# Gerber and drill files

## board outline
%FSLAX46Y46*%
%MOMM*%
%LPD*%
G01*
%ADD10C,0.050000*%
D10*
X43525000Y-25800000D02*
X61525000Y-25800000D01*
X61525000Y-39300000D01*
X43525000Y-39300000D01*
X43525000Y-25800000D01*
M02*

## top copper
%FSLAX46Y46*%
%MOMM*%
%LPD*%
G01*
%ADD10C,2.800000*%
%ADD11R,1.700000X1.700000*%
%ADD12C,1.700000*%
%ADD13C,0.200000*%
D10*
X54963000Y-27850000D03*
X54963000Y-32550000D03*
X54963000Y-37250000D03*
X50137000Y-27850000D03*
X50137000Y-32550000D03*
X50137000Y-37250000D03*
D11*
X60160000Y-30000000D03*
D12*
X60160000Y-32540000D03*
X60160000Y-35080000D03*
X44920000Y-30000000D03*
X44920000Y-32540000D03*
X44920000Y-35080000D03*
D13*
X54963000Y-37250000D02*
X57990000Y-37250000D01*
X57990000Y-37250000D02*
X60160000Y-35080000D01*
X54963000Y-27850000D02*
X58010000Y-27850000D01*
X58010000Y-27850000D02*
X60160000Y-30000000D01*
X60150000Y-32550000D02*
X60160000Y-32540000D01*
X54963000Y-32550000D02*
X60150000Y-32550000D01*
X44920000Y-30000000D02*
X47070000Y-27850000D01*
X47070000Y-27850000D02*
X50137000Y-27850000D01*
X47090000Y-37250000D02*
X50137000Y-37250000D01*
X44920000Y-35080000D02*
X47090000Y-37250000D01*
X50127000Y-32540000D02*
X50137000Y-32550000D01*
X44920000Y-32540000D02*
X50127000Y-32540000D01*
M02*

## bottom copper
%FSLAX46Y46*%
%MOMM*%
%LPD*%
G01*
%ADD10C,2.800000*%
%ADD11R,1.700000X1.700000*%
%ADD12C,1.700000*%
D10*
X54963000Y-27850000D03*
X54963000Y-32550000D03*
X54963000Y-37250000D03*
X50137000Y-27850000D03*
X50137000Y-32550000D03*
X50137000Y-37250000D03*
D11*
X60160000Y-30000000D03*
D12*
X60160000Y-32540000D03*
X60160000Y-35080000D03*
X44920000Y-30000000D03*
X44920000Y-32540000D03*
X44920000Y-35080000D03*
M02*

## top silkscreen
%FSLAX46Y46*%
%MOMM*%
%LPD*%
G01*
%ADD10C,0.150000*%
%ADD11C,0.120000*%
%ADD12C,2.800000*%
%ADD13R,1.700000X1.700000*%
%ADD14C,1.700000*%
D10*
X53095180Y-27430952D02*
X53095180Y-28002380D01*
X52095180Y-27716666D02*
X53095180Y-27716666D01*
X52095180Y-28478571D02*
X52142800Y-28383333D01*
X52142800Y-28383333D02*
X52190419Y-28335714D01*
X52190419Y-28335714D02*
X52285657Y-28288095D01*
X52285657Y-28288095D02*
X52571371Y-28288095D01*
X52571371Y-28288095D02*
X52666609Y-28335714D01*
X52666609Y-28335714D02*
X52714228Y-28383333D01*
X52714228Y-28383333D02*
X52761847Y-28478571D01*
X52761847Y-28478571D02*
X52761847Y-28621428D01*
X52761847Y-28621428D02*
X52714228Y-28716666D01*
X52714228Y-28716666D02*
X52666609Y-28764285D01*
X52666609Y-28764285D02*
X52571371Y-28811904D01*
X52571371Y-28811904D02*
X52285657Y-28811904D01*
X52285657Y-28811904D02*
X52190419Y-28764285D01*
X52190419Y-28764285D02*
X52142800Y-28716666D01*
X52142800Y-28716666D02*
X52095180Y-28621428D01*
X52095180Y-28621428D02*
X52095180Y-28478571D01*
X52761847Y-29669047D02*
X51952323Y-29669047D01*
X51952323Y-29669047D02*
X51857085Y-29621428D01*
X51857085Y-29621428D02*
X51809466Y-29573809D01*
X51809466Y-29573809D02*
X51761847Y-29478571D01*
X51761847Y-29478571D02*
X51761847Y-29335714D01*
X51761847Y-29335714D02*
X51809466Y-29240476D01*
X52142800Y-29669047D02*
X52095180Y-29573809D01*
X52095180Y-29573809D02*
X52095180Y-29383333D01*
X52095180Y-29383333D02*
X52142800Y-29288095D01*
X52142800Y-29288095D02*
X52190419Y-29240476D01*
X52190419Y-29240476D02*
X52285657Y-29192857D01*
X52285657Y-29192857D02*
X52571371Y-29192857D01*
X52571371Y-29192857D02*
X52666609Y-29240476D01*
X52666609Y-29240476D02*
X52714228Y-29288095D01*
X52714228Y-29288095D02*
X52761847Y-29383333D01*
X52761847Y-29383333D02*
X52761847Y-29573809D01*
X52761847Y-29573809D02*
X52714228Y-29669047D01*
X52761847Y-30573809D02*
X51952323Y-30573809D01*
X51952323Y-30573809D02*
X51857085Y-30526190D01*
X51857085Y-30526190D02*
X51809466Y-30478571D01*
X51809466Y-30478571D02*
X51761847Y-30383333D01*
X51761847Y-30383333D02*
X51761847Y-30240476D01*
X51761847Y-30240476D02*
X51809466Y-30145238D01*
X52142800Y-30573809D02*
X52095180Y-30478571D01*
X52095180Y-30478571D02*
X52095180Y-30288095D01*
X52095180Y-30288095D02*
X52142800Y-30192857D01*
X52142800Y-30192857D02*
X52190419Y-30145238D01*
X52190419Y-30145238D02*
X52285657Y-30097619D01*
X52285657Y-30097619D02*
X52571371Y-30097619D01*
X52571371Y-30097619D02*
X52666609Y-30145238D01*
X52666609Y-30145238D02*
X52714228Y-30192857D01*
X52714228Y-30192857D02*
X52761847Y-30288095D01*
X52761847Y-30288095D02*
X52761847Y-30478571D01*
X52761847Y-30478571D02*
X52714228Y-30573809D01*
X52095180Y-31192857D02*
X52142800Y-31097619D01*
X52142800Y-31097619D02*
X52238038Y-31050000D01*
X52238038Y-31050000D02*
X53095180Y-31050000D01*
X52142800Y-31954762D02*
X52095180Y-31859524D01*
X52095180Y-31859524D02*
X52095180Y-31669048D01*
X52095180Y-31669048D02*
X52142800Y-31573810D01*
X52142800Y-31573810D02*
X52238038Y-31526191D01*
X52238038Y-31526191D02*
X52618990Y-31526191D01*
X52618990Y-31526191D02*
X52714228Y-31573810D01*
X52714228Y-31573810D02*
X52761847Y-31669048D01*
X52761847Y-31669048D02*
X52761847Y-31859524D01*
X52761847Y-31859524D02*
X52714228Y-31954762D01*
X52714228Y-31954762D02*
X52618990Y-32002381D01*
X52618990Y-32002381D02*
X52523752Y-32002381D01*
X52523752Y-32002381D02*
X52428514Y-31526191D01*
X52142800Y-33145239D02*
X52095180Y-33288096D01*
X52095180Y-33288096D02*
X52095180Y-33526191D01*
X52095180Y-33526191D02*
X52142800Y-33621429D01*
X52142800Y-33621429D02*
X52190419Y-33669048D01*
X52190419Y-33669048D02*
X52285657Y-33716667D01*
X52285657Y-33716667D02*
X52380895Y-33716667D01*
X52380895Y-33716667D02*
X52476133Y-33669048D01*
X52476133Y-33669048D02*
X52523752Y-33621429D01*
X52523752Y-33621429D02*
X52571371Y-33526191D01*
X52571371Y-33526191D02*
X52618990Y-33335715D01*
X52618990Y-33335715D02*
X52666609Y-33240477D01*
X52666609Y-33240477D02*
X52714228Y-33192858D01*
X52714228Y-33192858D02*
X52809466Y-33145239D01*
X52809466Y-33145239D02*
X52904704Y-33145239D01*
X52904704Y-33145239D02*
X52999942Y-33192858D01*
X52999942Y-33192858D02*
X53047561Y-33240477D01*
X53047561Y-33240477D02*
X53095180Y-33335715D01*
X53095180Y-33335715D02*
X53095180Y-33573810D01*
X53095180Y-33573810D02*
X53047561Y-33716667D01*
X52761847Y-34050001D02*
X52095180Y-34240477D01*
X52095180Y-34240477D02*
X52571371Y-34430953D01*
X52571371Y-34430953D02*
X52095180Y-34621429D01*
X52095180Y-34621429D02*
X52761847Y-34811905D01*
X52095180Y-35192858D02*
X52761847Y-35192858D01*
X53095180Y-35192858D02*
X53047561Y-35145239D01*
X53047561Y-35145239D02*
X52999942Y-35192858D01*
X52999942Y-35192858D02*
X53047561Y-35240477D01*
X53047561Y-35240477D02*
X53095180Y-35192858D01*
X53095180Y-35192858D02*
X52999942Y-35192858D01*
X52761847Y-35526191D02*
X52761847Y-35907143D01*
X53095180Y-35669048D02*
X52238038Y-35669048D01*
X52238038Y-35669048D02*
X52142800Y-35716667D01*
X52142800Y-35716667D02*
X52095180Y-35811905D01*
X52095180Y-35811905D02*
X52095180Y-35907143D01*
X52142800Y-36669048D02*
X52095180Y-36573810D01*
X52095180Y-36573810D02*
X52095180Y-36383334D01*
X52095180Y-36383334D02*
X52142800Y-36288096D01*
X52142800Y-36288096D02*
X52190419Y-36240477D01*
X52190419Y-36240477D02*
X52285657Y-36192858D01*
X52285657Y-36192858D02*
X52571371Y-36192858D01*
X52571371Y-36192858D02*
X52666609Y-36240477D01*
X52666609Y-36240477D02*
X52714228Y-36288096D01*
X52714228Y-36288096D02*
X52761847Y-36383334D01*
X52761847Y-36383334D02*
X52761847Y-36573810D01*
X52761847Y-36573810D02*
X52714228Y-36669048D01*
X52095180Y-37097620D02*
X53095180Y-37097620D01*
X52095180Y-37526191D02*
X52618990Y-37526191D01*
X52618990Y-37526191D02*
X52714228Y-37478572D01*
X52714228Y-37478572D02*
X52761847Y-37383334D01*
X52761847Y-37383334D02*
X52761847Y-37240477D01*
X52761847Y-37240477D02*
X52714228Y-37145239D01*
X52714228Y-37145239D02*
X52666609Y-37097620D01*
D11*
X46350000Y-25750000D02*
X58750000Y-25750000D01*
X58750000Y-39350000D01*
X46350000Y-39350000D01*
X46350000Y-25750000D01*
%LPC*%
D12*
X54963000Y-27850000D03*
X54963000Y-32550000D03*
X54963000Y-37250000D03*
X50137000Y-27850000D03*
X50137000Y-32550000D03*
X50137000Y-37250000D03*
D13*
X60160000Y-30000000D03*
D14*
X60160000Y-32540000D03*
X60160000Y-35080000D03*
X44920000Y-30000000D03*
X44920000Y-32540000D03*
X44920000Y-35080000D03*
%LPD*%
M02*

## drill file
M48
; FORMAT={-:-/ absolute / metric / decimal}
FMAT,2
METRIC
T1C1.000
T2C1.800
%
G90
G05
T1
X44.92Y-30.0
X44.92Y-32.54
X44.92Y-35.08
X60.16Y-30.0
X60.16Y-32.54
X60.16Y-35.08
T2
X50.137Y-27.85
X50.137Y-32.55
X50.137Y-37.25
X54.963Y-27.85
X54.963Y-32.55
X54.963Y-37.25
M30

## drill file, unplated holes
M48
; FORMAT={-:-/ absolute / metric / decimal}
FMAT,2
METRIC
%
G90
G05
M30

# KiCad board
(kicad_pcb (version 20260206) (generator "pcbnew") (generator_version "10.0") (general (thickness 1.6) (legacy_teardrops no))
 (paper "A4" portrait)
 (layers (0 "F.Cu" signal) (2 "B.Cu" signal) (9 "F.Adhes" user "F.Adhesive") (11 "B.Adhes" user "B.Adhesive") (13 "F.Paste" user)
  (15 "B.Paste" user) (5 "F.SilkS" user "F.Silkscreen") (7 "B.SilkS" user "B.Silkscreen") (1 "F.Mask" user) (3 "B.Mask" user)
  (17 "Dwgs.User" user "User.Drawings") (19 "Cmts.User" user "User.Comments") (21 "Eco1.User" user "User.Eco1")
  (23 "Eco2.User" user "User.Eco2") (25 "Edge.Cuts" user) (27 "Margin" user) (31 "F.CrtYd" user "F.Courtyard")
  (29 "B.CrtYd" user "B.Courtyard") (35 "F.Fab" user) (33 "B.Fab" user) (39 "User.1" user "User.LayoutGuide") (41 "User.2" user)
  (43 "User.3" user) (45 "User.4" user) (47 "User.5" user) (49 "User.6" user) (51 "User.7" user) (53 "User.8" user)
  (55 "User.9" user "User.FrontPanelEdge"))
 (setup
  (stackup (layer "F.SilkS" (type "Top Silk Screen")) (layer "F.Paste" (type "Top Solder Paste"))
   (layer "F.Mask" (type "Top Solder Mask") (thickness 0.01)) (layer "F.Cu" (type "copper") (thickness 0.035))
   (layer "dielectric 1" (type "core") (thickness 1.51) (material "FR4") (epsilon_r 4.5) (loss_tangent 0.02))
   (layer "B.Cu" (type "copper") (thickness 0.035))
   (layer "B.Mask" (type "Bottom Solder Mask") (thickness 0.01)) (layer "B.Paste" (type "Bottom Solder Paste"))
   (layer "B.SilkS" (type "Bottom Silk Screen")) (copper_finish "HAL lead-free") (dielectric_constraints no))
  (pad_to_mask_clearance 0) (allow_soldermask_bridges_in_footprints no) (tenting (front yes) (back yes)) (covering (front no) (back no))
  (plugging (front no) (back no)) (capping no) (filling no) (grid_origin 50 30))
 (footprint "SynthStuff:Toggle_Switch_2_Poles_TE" (layer "F.Cu") (at 52.55 32.55 180)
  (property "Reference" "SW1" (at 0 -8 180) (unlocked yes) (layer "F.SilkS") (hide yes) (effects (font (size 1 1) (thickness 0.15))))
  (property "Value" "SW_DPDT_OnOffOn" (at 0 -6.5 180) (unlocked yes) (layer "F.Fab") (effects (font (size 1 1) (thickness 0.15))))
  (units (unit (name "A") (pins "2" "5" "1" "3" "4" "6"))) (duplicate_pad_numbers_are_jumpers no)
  (fp_rect (start -6.2 -6.8) (end 6.2 6.8) (stroke (width 0.12) (type default)) (fill no) (layer "F.SilkS"))
  (pad "1" thru_hole circle (at -2.413 4.7 270) (size 2.8 2.8) (drill 1.8) (layers "*.Cu" "*.Mask") (remove_unused_layers no)
   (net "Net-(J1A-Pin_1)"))
  (pad "2" thru_hole circle (at -2.413 0 270) (size 2.8 2.8) (drill 1.8) (layers "*.Cu" "*.Mask") (remove_unused_layers no)
   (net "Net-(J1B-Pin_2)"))
  (pad "3" thru_hole circle (at -2.413 -4.7 270) (size 2.8 2.8) (drill 1.8) (layers "*.Cu" "*.Mask") (remove_unused_layers no)
   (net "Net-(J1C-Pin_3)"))
  (pad "4" thru_hole circle (at 2.413 4.7 270) (size 2.8 2.8) (drill 1.8) (layers "*.Cu" "*.Mask") (remove_unused_layers no)
   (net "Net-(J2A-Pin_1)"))
  (pad "5" thru_hole circle (at 2.413 0 270) (size 2.8 2.8) (drill 1.8) (layers "*.Cu" "*.Mask") (remove_unused_layers no)
   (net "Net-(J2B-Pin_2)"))
  (pad "6" thru_hole circle (at 2.413 -4.7 270) (size 2.8 2.8) (drill 1.8) (layers "*.Cu" "*.Mask") (remove_unused_layers no)
   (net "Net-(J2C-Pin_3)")))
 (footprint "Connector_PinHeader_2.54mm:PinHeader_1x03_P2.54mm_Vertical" (layer "B.Cu") (at 60.16 30 180)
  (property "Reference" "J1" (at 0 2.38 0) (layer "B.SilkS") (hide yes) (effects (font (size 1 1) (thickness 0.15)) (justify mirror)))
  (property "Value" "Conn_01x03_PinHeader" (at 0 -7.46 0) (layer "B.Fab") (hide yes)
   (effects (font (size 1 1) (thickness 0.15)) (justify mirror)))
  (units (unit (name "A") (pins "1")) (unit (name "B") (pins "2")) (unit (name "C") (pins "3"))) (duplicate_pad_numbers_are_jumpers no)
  (pad "1" thru_hole rect (at 0 0 180) (size 1.7 1.7) (drill 1) (layers "*.Cu" "*.Mask") (remove_unused_layers no) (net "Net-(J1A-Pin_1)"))
  (pad "2" thru_hole circle (at 0 -2.54 180) (size 1.7 1.7) (drill 1) (layers "*.Cu" "*.Mask") (remove_unused_layers no)
   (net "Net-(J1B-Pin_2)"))
  (pad "3" thru_hole circle (at 0 -5.08 180) (size 1.7 1.7) (drill 1) (layers "*.Cu" "*.Mask") (remove_unused_layers no)
   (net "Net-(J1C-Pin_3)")))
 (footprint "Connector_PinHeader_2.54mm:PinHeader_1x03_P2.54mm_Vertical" (layer "B.Cu") (at 44.92 30 180)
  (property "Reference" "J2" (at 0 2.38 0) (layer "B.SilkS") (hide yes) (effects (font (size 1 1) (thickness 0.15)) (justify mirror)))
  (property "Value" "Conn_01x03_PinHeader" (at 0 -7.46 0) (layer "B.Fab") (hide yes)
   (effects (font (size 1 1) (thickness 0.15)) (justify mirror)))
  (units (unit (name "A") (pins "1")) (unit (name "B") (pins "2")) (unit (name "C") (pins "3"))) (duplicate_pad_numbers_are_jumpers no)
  (pad "1" thru_hole circle (at 0 0 180) (size 1.7 1.7) (drill 1) (layers "*.Cu" "*.Mask") (remove_unused_layers no) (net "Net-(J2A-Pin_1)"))
  (pad "2" thru_hole circle (at 0 -2.54 180) (size 1.7 1.7) (drill 1) (layers "*.Cu" "*.Mask") (remove_unused_layers no)
   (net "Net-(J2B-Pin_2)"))
  (pad "3" thru_hole circle (at 0 -5.08 180) (size 1.7 1.7) (drill 1) (layers "*.Cu" "*.Mask") (remove_unused_layers no)
   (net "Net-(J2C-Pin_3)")))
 (gr_rect (start 43.525 25.8) (end 61.525 39.3) (stroke (width 0.05) (type solid)) (fill no) (layer "Edge.Cuts"))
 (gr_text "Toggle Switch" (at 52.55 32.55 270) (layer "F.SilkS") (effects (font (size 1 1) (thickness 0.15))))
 (segment (start 54.963 27.85) (end 58.01 27.85) (width 0.2) (layer "F.Cu") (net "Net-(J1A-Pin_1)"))
 (segment (start 58.01 27.85) (end 60.16 30) (width 0.2) (layer "F.Cu") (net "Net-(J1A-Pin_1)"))
 (segment (start 60.15 32.55) (end 60.16 32.54) (width 0.2) (layer "F.Cu") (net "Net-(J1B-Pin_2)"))
 (segment (start 54.963 32.55) (end 60.15 32.55) (width 0.2) (layer "F.Cu") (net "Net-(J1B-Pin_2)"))
 (segment (start 54.963 37.25) (end 57.99 37.25) (width 0.2) (layer "F.Cu") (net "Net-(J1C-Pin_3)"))
 (segment (start 57.99 37.25) (end 60.16 35.08) (width 0.2) (layer "F.Cu") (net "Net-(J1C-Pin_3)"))
 (segment (start 44.92 30) (end 47.07 27.85) (width 0.2) (layer "F.Cu") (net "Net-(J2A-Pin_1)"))
 (segment (start 47.07 27.85) (end 50.137 27.85) (width 0.2) (layer "F.Cu") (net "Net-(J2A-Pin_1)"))
 (segment (start 50.127 32.54) (end 50.137 32.55) (width 0.2) (layer "F.Cu") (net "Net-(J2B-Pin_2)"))
 (segment (start 44.92 32.54) (end 50.127 32.54) (width 0.2) (layer "F.Cu") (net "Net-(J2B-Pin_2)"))
 (segment (start 47.09 37.25) (end 50.137 37.25) (width 0.2) (layer "F.Cu") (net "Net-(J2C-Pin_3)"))
 (segment (start 44.92 35.08) (end 47.09 37.25) (width 0.2) (layer "F.Cu") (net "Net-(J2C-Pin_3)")))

